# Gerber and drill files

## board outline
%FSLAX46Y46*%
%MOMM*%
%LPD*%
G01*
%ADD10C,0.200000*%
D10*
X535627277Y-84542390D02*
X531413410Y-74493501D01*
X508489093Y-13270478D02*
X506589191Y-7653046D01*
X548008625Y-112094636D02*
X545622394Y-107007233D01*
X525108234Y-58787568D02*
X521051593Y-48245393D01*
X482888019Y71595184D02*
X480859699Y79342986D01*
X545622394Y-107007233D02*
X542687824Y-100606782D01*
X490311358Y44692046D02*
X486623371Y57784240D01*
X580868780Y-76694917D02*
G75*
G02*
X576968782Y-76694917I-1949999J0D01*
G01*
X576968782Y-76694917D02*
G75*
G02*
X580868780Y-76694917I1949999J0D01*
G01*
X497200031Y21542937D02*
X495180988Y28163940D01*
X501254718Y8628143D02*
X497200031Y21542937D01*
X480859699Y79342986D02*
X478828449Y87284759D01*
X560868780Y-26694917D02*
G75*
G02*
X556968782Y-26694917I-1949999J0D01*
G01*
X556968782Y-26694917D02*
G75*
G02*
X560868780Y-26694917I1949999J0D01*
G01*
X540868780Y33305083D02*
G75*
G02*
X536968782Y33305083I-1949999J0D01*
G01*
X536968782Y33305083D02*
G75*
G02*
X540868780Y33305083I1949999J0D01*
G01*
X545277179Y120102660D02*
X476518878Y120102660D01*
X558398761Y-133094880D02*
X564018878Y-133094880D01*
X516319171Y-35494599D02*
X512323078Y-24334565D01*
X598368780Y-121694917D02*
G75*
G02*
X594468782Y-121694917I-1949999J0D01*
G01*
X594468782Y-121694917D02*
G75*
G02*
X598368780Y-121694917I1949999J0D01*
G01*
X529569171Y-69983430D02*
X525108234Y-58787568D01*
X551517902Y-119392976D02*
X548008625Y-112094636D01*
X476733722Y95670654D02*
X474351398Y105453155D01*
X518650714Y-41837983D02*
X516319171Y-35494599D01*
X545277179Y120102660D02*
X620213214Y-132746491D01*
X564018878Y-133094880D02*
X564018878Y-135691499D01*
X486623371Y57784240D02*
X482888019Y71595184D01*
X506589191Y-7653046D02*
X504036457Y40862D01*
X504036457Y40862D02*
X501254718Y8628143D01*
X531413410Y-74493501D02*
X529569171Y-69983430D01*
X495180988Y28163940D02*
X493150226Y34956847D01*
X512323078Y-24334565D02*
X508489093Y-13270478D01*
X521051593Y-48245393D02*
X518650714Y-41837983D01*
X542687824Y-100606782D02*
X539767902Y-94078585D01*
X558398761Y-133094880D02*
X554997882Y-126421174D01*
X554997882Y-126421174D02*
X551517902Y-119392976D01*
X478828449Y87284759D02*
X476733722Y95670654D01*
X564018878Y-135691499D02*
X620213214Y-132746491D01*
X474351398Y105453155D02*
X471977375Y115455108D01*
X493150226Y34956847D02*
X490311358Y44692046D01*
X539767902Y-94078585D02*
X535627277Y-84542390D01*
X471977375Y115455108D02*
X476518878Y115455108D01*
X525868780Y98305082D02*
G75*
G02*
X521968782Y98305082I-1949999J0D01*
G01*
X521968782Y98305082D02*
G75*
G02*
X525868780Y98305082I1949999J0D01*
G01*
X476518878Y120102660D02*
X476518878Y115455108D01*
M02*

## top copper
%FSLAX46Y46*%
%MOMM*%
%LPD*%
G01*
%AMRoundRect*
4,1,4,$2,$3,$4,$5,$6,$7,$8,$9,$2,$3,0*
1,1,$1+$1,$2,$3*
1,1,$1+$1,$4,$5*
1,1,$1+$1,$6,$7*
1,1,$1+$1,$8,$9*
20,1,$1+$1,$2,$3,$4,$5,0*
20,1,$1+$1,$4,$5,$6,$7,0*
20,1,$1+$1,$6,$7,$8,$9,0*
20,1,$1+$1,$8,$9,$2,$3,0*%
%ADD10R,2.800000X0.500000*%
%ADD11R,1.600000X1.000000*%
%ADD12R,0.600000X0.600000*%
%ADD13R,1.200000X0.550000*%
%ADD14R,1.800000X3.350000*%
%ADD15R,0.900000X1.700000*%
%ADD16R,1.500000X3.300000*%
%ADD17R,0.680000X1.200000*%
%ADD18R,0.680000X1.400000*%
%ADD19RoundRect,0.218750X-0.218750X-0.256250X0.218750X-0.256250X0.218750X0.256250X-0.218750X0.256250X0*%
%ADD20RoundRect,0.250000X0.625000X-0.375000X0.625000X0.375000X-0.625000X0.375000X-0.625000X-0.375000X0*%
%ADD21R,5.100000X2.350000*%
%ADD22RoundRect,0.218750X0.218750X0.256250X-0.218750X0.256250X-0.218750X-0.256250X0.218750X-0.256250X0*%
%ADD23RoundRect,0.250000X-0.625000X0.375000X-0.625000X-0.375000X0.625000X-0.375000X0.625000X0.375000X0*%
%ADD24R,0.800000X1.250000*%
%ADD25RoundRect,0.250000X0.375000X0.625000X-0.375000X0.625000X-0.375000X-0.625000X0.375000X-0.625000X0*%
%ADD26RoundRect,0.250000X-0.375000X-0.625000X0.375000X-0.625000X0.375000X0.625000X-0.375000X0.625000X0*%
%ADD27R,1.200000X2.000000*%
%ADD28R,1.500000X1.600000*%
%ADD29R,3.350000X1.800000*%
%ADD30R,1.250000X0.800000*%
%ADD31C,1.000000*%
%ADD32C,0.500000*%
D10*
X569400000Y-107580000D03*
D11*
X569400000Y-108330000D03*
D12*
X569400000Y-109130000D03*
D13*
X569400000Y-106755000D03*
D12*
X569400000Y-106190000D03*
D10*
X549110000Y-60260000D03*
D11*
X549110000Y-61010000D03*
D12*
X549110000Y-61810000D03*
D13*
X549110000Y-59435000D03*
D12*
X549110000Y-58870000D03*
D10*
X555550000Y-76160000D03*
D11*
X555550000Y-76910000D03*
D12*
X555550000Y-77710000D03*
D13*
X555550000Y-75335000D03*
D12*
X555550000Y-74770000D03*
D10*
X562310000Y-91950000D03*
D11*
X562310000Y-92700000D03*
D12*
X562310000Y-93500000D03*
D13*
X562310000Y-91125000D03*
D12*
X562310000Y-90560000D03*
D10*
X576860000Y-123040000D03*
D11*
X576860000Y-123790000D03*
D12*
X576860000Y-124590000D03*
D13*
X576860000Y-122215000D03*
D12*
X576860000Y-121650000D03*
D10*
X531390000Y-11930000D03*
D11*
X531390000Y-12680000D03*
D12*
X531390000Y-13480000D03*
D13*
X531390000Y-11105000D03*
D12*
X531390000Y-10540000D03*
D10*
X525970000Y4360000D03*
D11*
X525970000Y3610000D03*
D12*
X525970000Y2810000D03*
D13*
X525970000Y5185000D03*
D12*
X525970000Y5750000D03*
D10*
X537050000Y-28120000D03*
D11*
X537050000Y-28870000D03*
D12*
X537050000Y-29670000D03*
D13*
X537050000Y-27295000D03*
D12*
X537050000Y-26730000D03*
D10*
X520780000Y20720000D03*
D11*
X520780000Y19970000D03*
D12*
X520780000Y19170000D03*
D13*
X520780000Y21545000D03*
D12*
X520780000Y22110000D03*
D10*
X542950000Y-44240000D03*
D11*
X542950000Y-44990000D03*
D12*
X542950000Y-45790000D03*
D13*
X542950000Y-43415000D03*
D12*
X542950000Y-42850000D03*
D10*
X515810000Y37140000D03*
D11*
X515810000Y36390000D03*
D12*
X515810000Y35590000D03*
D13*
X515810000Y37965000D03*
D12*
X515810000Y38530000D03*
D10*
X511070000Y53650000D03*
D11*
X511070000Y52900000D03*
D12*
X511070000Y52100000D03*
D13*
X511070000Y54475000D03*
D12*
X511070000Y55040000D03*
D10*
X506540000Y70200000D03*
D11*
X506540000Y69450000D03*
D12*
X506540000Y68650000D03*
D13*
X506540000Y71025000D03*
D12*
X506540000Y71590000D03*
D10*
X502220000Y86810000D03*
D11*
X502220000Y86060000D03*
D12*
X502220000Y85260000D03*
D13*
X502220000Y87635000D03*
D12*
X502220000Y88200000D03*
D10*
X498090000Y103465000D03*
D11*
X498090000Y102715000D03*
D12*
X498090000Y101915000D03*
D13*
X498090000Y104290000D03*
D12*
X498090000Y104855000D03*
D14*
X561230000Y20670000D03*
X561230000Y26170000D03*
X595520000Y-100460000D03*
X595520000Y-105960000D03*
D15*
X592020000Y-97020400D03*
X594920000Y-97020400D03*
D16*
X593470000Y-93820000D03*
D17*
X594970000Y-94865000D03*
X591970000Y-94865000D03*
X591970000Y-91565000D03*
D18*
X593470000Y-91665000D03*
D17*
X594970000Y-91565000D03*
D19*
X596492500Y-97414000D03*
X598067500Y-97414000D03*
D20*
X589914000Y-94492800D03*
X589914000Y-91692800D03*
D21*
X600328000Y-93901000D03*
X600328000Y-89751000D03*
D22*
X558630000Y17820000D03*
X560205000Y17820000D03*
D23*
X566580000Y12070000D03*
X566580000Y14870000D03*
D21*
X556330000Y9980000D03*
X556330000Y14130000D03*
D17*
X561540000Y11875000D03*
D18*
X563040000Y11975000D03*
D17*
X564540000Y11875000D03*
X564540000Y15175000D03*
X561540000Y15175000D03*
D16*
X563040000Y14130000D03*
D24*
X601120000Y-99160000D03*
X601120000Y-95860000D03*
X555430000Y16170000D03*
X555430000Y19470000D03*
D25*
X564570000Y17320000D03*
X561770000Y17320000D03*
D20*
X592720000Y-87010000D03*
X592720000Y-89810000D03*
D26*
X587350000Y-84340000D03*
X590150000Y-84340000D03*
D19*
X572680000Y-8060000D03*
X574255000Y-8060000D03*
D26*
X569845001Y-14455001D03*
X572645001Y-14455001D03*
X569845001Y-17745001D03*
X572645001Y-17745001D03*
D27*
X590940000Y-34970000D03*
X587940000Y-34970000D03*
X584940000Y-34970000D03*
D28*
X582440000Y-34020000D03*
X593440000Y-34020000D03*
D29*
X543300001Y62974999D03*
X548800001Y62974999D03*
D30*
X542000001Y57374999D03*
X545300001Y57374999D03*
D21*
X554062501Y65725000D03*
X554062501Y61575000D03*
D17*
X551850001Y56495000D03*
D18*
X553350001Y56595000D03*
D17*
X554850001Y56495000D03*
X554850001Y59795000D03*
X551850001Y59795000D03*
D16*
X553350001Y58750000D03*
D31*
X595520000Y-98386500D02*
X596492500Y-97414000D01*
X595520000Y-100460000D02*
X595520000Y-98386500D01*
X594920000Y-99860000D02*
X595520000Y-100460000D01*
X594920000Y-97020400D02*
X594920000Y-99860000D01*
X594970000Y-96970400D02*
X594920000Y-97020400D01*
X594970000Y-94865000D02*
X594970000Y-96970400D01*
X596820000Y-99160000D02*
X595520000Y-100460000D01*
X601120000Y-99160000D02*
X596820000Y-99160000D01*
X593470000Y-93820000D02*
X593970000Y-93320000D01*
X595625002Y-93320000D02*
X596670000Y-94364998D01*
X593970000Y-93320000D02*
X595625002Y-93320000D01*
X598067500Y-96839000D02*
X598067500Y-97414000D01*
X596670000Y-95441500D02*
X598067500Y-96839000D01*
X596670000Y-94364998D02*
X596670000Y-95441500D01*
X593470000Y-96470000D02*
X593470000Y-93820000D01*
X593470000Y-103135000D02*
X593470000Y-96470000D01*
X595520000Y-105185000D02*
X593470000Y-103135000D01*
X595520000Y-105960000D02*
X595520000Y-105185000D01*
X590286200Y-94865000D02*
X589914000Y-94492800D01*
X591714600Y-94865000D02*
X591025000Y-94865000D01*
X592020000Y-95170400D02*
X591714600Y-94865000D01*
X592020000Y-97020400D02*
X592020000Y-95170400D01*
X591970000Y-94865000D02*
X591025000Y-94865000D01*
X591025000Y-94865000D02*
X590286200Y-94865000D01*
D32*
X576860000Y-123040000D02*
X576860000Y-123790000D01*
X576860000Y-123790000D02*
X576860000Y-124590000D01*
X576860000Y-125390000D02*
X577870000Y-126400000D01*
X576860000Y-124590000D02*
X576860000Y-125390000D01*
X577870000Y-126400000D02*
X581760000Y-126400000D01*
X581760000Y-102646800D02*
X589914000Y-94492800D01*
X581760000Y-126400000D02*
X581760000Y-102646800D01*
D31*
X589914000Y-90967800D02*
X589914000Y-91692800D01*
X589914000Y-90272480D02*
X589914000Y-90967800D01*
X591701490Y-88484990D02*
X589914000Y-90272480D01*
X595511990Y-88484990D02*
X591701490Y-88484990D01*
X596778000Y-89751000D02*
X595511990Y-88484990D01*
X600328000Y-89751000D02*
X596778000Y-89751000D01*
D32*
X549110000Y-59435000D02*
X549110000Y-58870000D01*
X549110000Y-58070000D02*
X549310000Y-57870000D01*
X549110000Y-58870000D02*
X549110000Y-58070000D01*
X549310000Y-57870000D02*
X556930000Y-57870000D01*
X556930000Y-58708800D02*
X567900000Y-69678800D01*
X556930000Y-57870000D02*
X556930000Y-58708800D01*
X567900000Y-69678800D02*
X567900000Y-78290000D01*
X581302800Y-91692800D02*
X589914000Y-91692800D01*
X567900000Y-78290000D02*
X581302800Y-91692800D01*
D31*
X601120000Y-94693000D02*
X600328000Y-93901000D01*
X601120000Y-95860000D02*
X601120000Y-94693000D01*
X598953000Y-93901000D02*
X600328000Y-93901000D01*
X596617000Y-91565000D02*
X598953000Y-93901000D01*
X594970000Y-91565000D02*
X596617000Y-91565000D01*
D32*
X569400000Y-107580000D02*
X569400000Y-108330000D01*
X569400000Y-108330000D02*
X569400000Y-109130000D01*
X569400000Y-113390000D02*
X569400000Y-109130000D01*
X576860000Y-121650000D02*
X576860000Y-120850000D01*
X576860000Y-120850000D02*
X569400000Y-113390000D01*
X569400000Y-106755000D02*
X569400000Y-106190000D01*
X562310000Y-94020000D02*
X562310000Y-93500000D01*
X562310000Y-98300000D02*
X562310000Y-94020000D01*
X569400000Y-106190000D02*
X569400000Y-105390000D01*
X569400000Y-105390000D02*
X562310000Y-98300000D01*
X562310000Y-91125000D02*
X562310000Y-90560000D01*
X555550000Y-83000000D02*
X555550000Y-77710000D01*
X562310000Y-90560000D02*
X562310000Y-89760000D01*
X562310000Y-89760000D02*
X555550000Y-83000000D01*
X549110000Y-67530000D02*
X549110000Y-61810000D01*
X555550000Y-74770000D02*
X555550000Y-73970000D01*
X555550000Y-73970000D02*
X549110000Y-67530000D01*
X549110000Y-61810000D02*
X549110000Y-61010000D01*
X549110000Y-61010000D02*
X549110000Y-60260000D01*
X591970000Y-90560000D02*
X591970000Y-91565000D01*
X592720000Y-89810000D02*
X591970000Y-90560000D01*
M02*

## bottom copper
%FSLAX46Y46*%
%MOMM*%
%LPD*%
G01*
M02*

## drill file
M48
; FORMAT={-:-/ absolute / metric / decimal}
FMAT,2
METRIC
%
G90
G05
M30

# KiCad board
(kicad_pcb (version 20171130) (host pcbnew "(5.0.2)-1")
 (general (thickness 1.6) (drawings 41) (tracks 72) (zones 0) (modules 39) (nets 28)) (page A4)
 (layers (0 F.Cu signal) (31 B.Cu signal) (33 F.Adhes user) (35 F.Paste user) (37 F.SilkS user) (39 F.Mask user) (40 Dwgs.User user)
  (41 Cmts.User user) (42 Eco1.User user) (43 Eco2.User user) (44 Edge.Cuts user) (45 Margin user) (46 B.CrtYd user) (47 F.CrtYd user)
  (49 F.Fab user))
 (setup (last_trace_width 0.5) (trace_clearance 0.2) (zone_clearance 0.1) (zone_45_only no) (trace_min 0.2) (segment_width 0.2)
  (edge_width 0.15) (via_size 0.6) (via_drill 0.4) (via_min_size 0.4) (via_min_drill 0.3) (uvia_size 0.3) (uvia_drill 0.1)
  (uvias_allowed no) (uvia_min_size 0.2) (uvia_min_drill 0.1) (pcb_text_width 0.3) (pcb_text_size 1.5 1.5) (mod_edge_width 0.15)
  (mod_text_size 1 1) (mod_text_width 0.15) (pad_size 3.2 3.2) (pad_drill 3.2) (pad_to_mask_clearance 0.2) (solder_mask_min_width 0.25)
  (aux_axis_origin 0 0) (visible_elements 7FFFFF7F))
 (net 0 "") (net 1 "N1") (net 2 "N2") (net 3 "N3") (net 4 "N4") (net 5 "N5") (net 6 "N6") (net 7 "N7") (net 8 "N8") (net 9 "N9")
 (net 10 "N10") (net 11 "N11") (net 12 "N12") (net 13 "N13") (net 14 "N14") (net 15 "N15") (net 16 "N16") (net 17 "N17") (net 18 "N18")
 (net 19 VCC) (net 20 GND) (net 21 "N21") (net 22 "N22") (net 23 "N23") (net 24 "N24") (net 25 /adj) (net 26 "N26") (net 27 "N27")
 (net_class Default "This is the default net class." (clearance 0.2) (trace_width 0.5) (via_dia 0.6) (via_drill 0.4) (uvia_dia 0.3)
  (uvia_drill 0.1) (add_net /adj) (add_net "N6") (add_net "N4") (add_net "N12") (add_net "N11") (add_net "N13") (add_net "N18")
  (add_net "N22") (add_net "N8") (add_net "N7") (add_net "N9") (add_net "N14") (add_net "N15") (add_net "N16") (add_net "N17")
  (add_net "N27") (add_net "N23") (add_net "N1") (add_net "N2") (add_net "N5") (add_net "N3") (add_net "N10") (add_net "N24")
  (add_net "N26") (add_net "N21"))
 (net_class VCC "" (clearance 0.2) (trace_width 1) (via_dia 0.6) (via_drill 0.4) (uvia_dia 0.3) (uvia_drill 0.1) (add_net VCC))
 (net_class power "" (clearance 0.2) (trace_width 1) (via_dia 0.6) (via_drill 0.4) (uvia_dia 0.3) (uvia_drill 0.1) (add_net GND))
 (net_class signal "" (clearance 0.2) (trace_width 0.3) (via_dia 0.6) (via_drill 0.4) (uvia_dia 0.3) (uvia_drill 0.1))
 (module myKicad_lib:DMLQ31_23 (layer F.Cu) (at 569.4 107.58 180)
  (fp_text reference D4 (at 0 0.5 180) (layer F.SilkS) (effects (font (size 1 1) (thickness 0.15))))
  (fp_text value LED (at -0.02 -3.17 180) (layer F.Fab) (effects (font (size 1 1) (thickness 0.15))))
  (pad 2 smd rect (at 0 0 180) (size 2.8 0.5) (layers F.Cu F.Paste F.Mask) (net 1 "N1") (zone_connect 2))
  (pad 2 smd rect (at 0 -0.75 180) (size 1.6 1) (layers F.Cu F.Paste F.Mask) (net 1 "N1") (zone_connect 2))
  (pad 2 smd rect (at 0 -1.55 180) (size 0.6 0.6) (layers F.Cu F.Paste F.Mask) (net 1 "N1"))
  (pad 1 smd rect (at 0 0.825 180) (size 1.2 0.55) (layers F.Cu F.Paste F.Mask) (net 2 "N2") (zone_connect 2))
  (pad 1 smd rect (at 0 1.39 180) (size 0.6 0.6) (layers F.Cu F.Paste F.Mask) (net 2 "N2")))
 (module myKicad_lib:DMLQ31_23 (layer F.Cu) (at 549.11 60.26 180)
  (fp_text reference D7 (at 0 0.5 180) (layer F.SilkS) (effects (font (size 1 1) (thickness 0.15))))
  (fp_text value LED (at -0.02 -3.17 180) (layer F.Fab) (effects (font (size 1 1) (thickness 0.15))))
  (pad 2 smd rect (at 0 0 180) (size 2.8 0.5) (layers F.Cu F.Paste F.Mask) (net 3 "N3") (zone_connect 2))
  (pad 2 smd rect (at 0 -0.75 180) (size 1.6 1) (layers F.Cu F.Paste F.Mask) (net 3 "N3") (zone_connect 2))
  (pad 2 smd rect (at 0 -1.55 180) (size 0.6 0.6) (layers F.Cu F.Paste F.Mask) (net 3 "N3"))
  (pad 1 smd rect (at 0 0.825 180) (size 1.2 0.55) (layers F.Cu F.Paste F.Mask) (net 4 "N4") (zone_connect 2))
  (pad 1 smd rect (at 0 1.39 180) (size 0.6 0.6) (layers F.Cu F.Paste F.Mask) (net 4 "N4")))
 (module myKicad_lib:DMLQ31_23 (layer F.Cu) (at 555.55 76.16 180)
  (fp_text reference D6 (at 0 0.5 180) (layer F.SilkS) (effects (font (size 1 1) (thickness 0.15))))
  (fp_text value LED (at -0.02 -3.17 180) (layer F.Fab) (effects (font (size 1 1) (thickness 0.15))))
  (pad 2 smd rect (at 0 0 180) (size 2.8 0.5) (layers F.Cu F.Paste F.Mask) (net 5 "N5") (zone_connect 2))
  (pad 2 smd rect (at 0 -0.75 180) (size 1.6 1) (layers F.Cu F.Paste F.Mask) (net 5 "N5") (zone_connect 2))
  (pad 2 smd rect (at 0 -1.55 180) (size 0.6 0.6) (layers F.Cu F.Paste F.Mask) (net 5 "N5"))
  (pad 1 smd rect (at 0 0.825 180) (size 1.2 0.55) (layers F.Cu F.Paste F.Mask) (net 3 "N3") (zone_connect 2))
  (pad 1 smd rect (at 0 1.39 180) (size 0.6 0.6) (layers F.Cu F.Paste F.Mask) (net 3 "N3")))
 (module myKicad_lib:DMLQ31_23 (layer F.Cu) (at 562.31 91.95 180)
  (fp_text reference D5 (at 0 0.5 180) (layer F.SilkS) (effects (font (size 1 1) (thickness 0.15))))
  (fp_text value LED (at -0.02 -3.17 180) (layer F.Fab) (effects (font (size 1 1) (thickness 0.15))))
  (pad 2 smd rect (at 0 0 180) (size 2.8 0.5) (layers F.Cu F.Paste F.Mask) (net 2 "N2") (zone_connect 2))
  (pad 2 smd rect (at 0 -0.75 180) (size 1.6 1) (layers F.Cu F.Paste F.Mask) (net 2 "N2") (zone_connect 2))
  (pad 2 smd rect (at 0 -1.55 180) (size 0.6 0.6) (layers F.Cu F.Paste F.Mask) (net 2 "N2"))
  (pad 1 smd rect (at 0 0.825 180) (size 1.2 0.55) (layers F.Cu F.Paste F.Mask) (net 5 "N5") (zone_connect 2))
  (pad 1 smd rect (at 0 1.39 180) (size 0.6 0.6) (layers F.Cu F.Paste F.Mask) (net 5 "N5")))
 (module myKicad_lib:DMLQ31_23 (layer F.Cu) (at 576.86 123.04 180)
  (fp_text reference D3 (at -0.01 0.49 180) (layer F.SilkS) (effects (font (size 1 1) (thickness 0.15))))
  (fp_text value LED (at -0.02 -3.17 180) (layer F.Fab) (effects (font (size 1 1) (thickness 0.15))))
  (pad 2 smd rect (at 0 0 180) (size 2.8 0.5) (layers F.Cu F.Paste F.Mask) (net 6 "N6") (zone_connect 2))
  (pad 2 smd rect (at 0 -0.75 180) (size 1.6 1) (layers F.Cu F.Paste F.Mask) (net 6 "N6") (zone_connect 2))
  (pad 2 smd rect (at 0 -1.55 180) (size 0.6 0.6) (layers F.Cu F.Paste F.Mask) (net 6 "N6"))
  (pad 1 smd rect (at 0 0.825 180) (size 1.2 0.55) (layers F.Cu F.Paste F.Mask) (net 1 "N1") (zone_connect 2))
  (pad 1 smd rect (at 0 1.39 180) (size 0.6 0.6) (layers F.Cu F.Paste F.Mask) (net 1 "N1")))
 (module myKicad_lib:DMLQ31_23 (layer F.Cu) (at 531.39 11.93 180)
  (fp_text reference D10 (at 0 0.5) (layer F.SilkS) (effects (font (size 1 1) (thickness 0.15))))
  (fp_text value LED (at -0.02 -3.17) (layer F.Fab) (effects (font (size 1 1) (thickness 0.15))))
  (pad 2 smd rect (at 0 0 180) (size 2.8 0.5) (layers F.Cu F.Paste F.Mask) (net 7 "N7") (zone_connect 2))
  (pad 2 smd rect (at 0 -0.75 180) (size 1.6 1) (layers F.Cu F.Paste F.Mask) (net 7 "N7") (zone_connect 2))
  (pad 2 smd rect (at 0 -1.55 180) (size 0.6 0.6) (layers F.Cu F.Paste F.Mask) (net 7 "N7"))
  (pad 1 smd rect (at 0 0.825 180) (size 1.2 0.55) (layers F.Cu F.Paste F.Mask) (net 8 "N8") (zone_connect 2))
  (pad 1 smd rect (at 0 1.39 180) (size 0.6 0.6) (layers F.Cu F.Paste F.Mask) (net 8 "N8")))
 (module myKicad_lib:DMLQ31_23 (layer F.Cu) (at 525.97 -4.36 180)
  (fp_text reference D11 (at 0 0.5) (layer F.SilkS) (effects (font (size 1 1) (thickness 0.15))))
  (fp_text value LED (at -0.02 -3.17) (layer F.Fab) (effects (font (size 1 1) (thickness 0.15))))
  (pad 2 smd rect (at 0 0 180) (size 2.8 0.5) (layers F.Cu F.Paste F.Mask) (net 8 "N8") (zone_connect 2))
  (pad 2 smd rect (at 0 -0.75 180) (size 1.6 1) (layers F.Cu F.Paste F.Mask) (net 8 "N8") (zone_connect 2))
  (pad 2 smd rect (at 0 -1.55 180) (size 0.6 0.6) (layers F.Cu F.Paste F.Mask) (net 8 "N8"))
  (pad 1 smd rect (at 0 0.825 180) (size 1.2 0.55) (layers F.Cu F.Paste F.Mask) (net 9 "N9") (zone_connect 2))
  (pad 1 smd rect (at 0 1.39 180) (size 0.6 0.6) (layers F.Cu F.Paste F.Mask) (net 9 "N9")))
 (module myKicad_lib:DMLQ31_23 (layer F.Cu) (at 537.05 28.12 180)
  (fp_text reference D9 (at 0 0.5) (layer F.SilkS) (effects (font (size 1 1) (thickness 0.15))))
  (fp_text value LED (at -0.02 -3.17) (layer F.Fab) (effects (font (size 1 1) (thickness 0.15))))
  (pad 2 smd rect (at 0 0 180) (size 2.8 0.5) (layers F.Cu F.Paste F.Mask) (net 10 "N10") (zone_connect 2))
  (pad 2 smd rect (at 0 -0.75 180) (size 1.6 1) (layers F.Cu F.Paste F.Mask) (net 10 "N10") (zone_connect 2))
  (pad 2 smd rect (at 0 -1.55 180) (size 0.6 0.6) (layers F.Cu F.Paste F.Mask) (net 10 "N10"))
  (pad 1 smd rect (at 0 0.825 180) (size 1.2 0.55) (layers F.Cu F.Paste F.Mask) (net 7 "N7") (zone_connect 2))
  (pad 1 smd rect (at 0 1.39 180) (size 0.6 0.6) (layers F.Cu F.Paste F.Mask) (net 7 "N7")))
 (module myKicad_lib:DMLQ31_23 (layer F.Cu) (at 520.78 -20.72 180)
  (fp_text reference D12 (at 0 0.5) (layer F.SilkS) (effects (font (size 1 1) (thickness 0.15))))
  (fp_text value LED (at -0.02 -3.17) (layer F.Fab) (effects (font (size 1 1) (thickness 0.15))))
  (pad 2 smd rect (at 0 0 180) (size 2.8 0.5) (layers F.Cu F.Paste F.Mask) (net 9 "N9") (zone_connect 2))
  (pad 2 smd rect (at 0 -0.75 180) (size 1.6 1) (layers F.Cu F.Paste F.Mask) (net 9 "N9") (zone_connect 2))
  (pad 2 smd rect (at 0 -1.55 180) (size 0.6 0.6) (layers F.Cu F.Paste F.Mask) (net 9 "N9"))
  (pad 1 smd rect (at 0 0.825 180) (size 1.2 0.55) (layers F.Cu F.Paste F.Mask) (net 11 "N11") (zone_connect 2))
  (pad 1 smd rect (at 0 1.39 180) (size 0.6 0.6) (layers F.Cu F.Paste F.Mask) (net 11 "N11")))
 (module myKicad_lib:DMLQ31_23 (layer F.Cu) (at 542.95 44.24 180)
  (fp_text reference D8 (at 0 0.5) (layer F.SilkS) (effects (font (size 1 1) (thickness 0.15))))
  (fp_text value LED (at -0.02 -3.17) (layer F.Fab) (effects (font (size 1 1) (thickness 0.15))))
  (pad 2 smd rect (at 0 0 180) (size 2.8 0.5) (layers F.Cu F.Paste F.Mask) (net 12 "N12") (zone_connect 2))
  (pad 2 smd rect (at 0 -0.75 180) (size 1.6 1) (layers F.Cu F.Paste F.Mask) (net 12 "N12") (zone_connect 2))
  (pad 2 smd rect (at 0 -1.55 180) (size 0.6 0.6) (layers F.Cu F.Paste F.Mask) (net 12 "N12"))
  (pad 1 smd rect (at 0 0.825 180) (size 1.2 0.55) (layers F.Cu F.Paste F.Mask) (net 10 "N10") (zone_connect 2))
  (pad 1 smd rect (at 0 1.39 180) (size 0.6 0.6) (layers F.Cu F.Paste F.Mask) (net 10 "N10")))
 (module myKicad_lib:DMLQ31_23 (layer F.Cu) (at 515.81 -37.14 180)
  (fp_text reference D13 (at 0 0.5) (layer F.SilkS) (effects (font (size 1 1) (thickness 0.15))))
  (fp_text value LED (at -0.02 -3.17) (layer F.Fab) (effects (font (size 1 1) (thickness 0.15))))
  (pad 2 smd rect (at 0 0 180) (size 2.8 0.5) (layers F.Cu F.Paste F.Mask) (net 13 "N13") (zone_connect 2))
  (pad 2 smd rect (at 0 -0.75 180) (size 1.6 1) (layers F.Cu F.Paste F.Mask) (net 13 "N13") (zone_connect 2))
  (pad 2 smd rect (at 0 -1.55 180) (size 0.6 0.6) (layers F.Cu F.Paste F.Mask) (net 13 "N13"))
  (pad 1 smd rect (at 0 0.825 180) (size 1.2 0.55) (layers F.Cu F.Paste F.Mask) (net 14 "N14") (zone_connect 2))
  (pad 1 smd rect (at 0 1.39 180) (size 0.6 0.6) (layers F.Cu F.Paste F.Mask) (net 14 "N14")))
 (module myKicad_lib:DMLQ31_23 (layer F.Cu) (at 511.07 -53.65 180)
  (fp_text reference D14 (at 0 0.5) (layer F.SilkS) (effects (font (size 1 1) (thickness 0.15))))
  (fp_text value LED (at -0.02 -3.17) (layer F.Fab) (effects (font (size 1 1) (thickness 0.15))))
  (pad 2 smd rect (at 0 0 180) (size 2.8 0.5) (layers F.Cu F.Paste F.Mask) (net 14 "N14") (zone_connect 2))
  (pad 2 smd rect (at 0 -0.75 180) (size 1.6 1) (layers F.Cu F.Paste F.Mask) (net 14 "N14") (zone_connect 2))
  (pad 2 smd rect (at 0 -1.55 180) (size 0.6 0.6) (layers F.Cu F.Paste F.Mask) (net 14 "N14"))
  (pad 1 smd rect (at 0 0.825 180) (size 1.2 0.55) (layers F.Cu F.Paste F.Mask) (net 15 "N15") (zone_connect 2))
  (pad 1 smd rect (at 0 1.39 180) (size 0.6 0.6) (layers F.Cu F.Paste F.Mask) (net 15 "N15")))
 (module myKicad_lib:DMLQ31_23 (layer F.Cu) (at 506.54 -70.2 180)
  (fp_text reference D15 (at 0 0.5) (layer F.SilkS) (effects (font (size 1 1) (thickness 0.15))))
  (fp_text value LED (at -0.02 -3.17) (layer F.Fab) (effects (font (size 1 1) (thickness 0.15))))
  (pad 2 smd rect (at 0 0 180) (size 2.8 0.5) (layers F.Cu F.Paste F.Mask) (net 15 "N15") (zone_connect 2))
  (pad 2 smd rect (at 0 -0.75 180) (size 1.6 1) (layers F.Cu F.Paste F.Mask) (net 15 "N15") (zone_connect 2))
  (pad 2 smd rect (at 0 -1.55 180) (size 0.6 0.6) (layers F.Cu F.Paste F.Mask) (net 15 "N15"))
  (pad 1 smd rect (at 0 0.825 180) (size 1.2 0.55) (layers F.Cu F.Paste F.Mask) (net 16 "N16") (zone_connect 2))
  (pad 1 smd rect (at 0 1.39 180) (size 0.6 0.6) (layers F.Cu F.Paste F.Mask) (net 16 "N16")))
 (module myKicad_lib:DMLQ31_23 (layer F.Cu) (at 502.22 -86.81 180)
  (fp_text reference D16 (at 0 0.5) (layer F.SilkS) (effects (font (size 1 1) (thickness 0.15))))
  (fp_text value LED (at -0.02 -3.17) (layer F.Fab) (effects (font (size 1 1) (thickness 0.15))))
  (pad 2 smd rect (at 0 0 180) (size 2.8 0.5) (layers F.Cu F.Paste F.Mask) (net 16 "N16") (zone_connect 2))
  (pad 2 smd rect (at 0 -0.75 180) (size 1.6 1) (layers F.Cu F.Paste F.Mask) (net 16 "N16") (zone_connect 2))
  (pad 2 smd rect (at 0 -1.55 180) (size 0.6 0.6) (layers F.Cu F.Paste F.Mask) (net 16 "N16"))
  (pad 1 smd rect (at 0 0.825 180) (size 1.2 0.55) (layers F.Cu F.Paste F.Mask) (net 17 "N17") (zone_connect 2))
  (pad 1 smd rect (at 0 1.39 180) (size 0.6 0.6) (layers F.Cu F.Paste F.Mask) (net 17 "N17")))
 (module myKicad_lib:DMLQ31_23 (layer F.Cu) (at 498.09 -103.465 180)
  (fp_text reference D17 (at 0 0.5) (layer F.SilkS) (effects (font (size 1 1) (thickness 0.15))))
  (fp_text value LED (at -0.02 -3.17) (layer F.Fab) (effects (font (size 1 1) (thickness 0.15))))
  (pad 2 smd rect (at 0 0 180) (size 2.8 0.5) (layers F.Cu F.Paste F.Mask) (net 17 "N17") (zone_connect 2))
  (pad 2 smd rect (at 0 -0.75 180) (size 1.6 1) (layers F.Cu F.Paste F.Mask) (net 17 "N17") (zone_connect 2))
  (pad 2 smd rect (at 0 -1.55 180) (size 0.6 0.6) (layers F.Cu F.Paste F.Mask) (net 17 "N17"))
  (pad 1 smd rect (at 0 0.825 180) (size 1.2 0.55) (layers F.Cu F.Paste F.Mask) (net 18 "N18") (zone_connect 2))
  (pad 1 smd rect (at 0 1.39 180) (size 0.6 0.6) (layers F.Cu F.Paste F.Mask) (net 18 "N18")))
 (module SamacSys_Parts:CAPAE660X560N (layer F.Cu) (at 561.23 -23.42 90)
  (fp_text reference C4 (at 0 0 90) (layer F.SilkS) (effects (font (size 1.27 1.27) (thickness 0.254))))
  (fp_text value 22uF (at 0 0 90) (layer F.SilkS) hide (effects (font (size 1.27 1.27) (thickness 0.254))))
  (pad 1 smd rect (at -2.75 0 180) (size 1.8 3.35) (layers F.Cu F.Paste F.Mask) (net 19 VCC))
  (pad 2 smd rect (at 2.75 0 180) (size 1.8 3.35) (layers F.Cu F.Paste F.Mask) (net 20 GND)))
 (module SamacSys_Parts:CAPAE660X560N (layer F.Cu) (at 595.52 103.21 270)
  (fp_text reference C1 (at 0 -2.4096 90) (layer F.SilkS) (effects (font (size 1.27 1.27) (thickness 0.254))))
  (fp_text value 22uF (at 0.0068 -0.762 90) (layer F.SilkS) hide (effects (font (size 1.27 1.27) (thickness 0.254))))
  (pad 1 smd rect (at -2.75 0) (size 1.8 3.35) (layers F.Cu F.Paste F.Mask) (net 19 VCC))
  (pad 2 smd rect (at 2.75 0) (size 1.8 3.35) (layers F.Cu F.Paste F.Mask) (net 20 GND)))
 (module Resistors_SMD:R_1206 (layer F.Cu) (at 593.47 97.0204)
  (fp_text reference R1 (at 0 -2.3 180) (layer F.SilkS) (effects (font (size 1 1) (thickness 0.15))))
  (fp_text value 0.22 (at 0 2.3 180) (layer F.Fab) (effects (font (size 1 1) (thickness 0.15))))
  (pad 1 smd rect (at -1.45 0) (size 0.9 1.7) (layers F.Cu F.Paste F.Mask) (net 6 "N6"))
  (pad 2 smd rect (at 1.45 0) (size 0.9 1.7) (layers F.Cu F.Paste F.Mask) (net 19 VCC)))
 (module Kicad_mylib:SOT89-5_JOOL (layer F.Cu) (at 593.47 93.215 180)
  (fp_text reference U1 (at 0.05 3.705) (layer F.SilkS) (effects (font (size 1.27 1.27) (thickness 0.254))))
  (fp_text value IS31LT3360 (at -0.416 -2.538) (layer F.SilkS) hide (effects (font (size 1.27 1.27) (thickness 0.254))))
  (pad 2 smd rect (at 0 -0.605 180) (size 1.5 3.3) (layers F.Cu F.Paste F.Mask) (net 20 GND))
  (pad 5 smd rect (at -1.5 -1.65 180) (size 0.68 1.2) (layers F.Cu F.Paste F.Mask) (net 19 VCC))
  (pad 4 smd rect (at 1.5 -1.65 180) (size 0.68 1.2) (layers F.Cu F.Paste F.Mask) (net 6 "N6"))
  (pad 3 smd rect (at 1.5 1.65 180) (size 0.68 1.2) (layers F.Cu F.Paste F.Mask) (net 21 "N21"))
  (pad 2 smd rect (at 0 1.55 180) (size 0.68 1.4) (layers F.Cu F.Paste F.Mask) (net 20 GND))
  (pad 1 smd rect (at -1.5 1.65 180) (size 0.68 1.2) (layers F.Cu F.Paste F.Mask) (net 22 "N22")))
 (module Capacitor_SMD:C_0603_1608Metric (layer F.Cu) (at 597.28 97.414)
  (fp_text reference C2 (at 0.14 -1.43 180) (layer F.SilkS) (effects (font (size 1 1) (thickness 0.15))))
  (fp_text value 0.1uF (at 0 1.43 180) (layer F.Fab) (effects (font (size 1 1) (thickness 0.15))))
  (pad 1 smd roundrect (at -0.7875 0) (size 0.875 0.95) (layers F.Cu F.Paste F.Mask) (roundrect_rratio 0.25) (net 19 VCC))
  (pad 2 smd roundrect (at 0.7875 0) (size 0.875 0.95) (layers F.Cu F.Paste F.Mask) (roundrect_rratio 0.25) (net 20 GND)))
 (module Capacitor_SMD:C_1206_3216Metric (layer F.Cu) (at 589.914 93.0928 90)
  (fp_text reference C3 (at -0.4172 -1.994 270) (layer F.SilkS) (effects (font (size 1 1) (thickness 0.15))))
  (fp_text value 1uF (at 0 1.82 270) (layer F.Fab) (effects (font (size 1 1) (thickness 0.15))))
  (pad 1 smd roundrect (at -1.4 0 90) (size 1.25 1.75) (layers F.Cu F.Paste F.Mask) (roundrect_rratio 0.2) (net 6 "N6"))
  (pad 2 smd roundrect (at 1.4 0 90) (size 1.25 1.75) (layers F.Cu F.Paste F.Mask) (roundrect_rratio 0.2) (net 4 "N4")))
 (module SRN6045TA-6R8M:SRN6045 (layer F.Cu) (at 600.328 91.826 180)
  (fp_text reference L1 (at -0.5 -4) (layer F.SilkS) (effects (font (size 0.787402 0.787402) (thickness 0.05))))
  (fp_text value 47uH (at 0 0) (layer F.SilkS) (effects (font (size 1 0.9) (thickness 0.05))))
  (pad 1 smd rect (at 0 -2.075 180) (size 5.1 2.35) (layers F.Cu F.Paste F.Mask) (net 22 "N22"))
  (pad 2 smd rect (at 0 2.075 180) (size 5.1 2.35) (layers F.Cu F.Paste F.Mask) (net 4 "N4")))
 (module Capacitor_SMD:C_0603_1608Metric (layer F.Cu) (at 559.4175 -17.82 180)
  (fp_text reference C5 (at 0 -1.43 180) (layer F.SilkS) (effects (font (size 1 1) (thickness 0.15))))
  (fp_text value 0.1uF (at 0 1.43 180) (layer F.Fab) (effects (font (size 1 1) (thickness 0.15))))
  (pad 2 smd roundrect (at 0.7875 0 180) (size 0.875 0.95) (layers F.Cu F.Paste F.Mask) (roundrect_rratio 0.25) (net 20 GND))
  (pad 1 smd roundrect (at -0.7875 0 180) (size 0.875 0.95) (layers F.Cu F.Paste F.Mask) (roundrect_rratio 0.25) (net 19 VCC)))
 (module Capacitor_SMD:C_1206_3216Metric (layer F.Cu) (at 566.58 -13.47 270)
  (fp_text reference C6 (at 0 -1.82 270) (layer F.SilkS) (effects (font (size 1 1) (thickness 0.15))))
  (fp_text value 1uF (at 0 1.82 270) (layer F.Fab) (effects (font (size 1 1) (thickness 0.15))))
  (pad 2 smd roundrect (at 1.4 0 270) (size 1.25 1.75) (layers F.Cu F.Paste F.Mask) (roundrect_rratio 0.2) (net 11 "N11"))
  (pad 1 smd roundrect (at -1.4 0 270) (size 1.25 1.75) (layers F.Cu F.Paste F.Mask) (roundrect_rratio 0.2) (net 12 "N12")))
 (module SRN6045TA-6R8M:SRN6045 (layer F.Cu) (at 556.33 -12.055)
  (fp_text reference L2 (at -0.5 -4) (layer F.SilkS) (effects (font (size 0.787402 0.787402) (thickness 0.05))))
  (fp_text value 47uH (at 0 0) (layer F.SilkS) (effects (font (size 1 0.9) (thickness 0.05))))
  (pad 2 smd rect (at 0 2.075) (size 5.1 2.35) (layers F.Cu F.Paste F.Mask) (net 11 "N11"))
  (pad 1 smd rect (at 0 -2.075) (size 5.1 2.35) (layers F.Cu F.Paste F.Mask) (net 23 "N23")))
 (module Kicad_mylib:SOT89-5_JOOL (layer F.Cu) (at 563.04 -13.525)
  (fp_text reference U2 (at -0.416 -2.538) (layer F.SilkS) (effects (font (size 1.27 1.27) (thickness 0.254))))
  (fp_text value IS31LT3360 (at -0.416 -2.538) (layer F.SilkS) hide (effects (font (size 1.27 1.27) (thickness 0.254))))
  (pad 1 smd rect (at -1.5 1.65) (size 0.68 1.2) (layers F.Cu F.Paste F.Mask) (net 23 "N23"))
  (pad 2 smd rect (at 0 1.55) (size 0.68 1.4) (layers F.Cu F.Paste F.Mask) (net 20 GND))
  (pad 3 smd rect (at 1.5 1.65) (size 0.68 1.2) (layers F.Cu F.Paste F.Mask) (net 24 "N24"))
  (pad 4 smd rect (at 1.5 -1.65) (size 0.68 1.2) (layers F.Cu F.Paste F.Mask) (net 12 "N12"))
  (pad 5 smd rect (at -1.5 -1.65) (size 0.68 1.2) (layers F.Cu F.Paste F.Mask) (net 19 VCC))
  (pad 2 smd rect (at 0 -0.605) (size 1.5 3.3) (layers F.Cu F.Paste F.Mask) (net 20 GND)))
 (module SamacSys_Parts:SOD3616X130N (layer F.Cu) (at 601.12 97.51 90)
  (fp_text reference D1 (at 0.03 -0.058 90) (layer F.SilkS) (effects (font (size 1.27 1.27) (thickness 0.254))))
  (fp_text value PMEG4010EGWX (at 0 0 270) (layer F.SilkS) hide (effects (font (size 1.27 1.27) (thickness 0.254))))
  (pad 1 smd rect (at -1.65 0 180) (size 0.8 1.25) (layers F.Cu F.Paste F.Mask) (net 19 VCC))
  (pad 2 smd rect (at 1.65 0 180) (size 0.8 1.25) (layers F.Cu F.Paste F.Mask) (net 22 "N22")))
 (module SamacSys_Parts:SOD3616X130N (layer F.Cu) (at 555.43 -17.82 270)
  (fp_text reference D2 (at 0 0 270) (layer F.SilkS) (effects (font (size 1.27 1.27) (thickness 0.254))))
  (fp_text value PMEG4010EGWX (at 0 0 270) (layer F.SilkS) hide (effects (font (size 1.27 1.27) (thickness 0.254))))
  (pad 2 smd rect (at 1.65 0) (size 0.8 1.25) (layers F.Cu F.Paste F.Mask) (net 23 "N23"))
  (pad 1 smd rect (at -1.65 0) (size 0.8 1.25) (layers F.Cu F.Paste F.Mask) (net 19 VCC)))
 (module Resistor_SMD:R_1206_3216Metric (layer F.Cu) (at 563.17 -17.32 180)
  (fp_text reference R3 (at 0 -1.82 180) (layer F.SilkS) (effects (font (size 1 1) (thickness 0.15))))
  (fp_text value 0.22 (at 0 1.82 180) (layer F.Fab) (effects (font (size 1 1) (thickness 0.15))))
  (pad 1 smd roundrect (at -1.4 0 180) (size 1.25 1.75) (layers F.Cu F.Paste F.Mask) (roundrect_rratio 0.2) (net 12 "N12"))
  (pad 2 smd roundrect (at 1.4 0 180) (size 1.25 1.75) (layers F.Cu F.Paste F.Mask) (roundrect_rratio 0.2) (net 19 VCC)))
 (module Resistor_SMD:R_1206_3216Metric (layer F.Cu) (at 592.72 88.41 90)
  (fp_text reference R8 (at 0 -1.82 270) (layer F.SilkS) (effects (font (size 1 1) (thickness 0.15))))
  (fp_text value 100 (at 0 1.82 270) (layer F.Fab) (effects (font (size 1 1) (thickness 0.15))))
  (pad 2 smd roundrect (at 1.4 0 90) (size 1.25 1.75) (layers F.Cu F.Paste F.Mask) (roundrect_rratio 0.2) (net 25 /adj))
  (pad 1 smd roundrect (at -1.4 0 90) (size 1.25 1.75) (layers F.Cu F.Paste F.Mask) (roundrect_rratio 0.2) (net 21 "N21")))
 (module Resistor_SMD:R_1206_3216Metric (layer F.Cu) (at 588.75 84.34)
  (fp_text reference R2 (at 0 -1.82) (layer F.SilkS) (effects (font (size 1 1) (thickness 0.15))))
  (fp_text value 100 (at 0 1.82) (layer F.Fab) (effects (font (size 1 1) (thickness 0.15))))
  (pad 1 smd roundrect (at -1.4 0) (size 1.25 1.75) (layers F.Cu F.Paste F.Mask) (roundrect_rratio 0.2) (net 24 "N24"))
  (pad 2 smd roundrect (at 1.4 0) (size 1.25 1.75) (layers F.Cu F.Paste F.Mask) (roundrect_rratio 0.2) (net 25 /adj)))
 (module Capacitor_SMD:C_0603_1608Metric (layer F.Cu) (at 573.4675 8.06)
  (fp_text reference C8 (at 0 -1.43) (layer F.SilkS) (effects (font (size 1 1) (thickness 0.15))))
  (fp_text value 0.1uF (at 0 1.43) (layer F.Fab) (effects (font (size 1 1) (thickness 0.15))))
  (pad 1 smd roundrect (at -0.7875 0) (size 0.875 0.95) (layers F.Cu F.Paste F.Mask) (roundrect_rratio 0.25) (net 19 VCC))
  (pad 2 smd roundrect (at 0.7875 0) (size 0.875 0.95) (layers F.Cu F.Paste F.Mask) (roundrect_rratio 0.25) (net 20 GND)))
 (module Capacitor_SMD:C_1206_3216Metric (layer F.Cu) (at 571.245001 14.455001)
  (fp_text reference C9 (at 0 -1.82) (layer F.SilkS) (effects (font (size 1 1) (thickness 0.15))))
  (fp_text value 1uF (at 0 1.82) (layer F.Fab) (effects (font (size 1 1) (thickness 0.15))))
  (pad 1 smd roundrect (at -1.4 0) (size 1.25 1.75) (layers F.Cu F.Paste F.Mask) (roundrect_rratio 0.2) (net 13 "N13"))
  (pad 2 smd roundrect (at 1.4 0) (size 1.25 1.75) (layers F.Cu F.Paste F.Mask) (roundrect_rratio 0.2) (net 18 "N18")))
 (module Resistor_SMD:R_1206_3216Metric (layer F.Cu) (at 571.245001 17.745001)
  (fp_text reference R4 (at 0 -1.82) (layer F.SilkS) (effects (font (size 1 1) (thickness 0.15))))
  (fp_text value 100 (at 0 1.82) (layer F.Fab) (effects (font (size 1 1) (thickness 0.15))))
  (pad 1 smd roundrect (at -1.4 0) (size 1.25 1.75) (layers F.Cu F.Paste F.Mask) (roundrect_rratio 0.2) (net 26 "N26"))
  (pad 2 smd roundrect (at 1.4 0) (size 1.25 1.75) (layers F.Cu F.Paste F.Mask) (roundrect_rratio 0.2) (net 25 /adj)))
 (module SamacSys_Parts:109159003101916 (layer F.Cu) (at 587.94 34.97)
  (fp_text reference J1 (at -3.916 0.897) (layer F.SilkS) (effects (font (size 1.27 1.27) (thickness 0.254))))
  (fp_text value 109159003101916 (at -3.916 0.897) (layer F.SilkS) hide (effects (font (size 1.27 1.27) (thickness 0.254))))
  (pad 1 smd rect (at 3 0) (size 1.2 2) (layers F.Cu F.Paste)) (pad 2 smd rect (at 0 0) (size 1.2 2) (layers F.Cu F.Paste))
  (pad 3 smd rect (at -3 0) (size 1.2 2) (layers F.Cu F.Paste))
  (pad 4 smd rect (at -5.5 -0.95) (size 1.5 1.6) (layers F.Cu F.Paste))
  (pad 5 smd rect (at 5.5 -0.95) (size 1.5 1.6) (layers F.Cu F.Paste)))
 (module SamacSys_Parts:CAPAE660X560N (layer F.Cu) (at 546.050001 -62.974999)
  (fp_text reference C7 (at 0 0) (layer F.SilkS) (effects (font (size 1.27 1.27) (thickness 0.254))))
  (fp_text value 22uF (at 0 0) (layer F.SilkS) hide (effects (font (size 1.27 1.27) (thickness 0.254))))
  (pad 1 smd rect (at -2.75 0 90) (size 1.8 3.35) (layers F.Cu F.Paste F.Mask) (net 19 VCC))
  (pad 2 smd rect (at 2.75 0 90) (size 1.8 3.35) (layers F.Cu F.Paste F.Mask) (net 20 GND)))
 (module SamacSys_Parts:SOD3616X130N (layer F.Cu) (at 543.650001 -57.374999)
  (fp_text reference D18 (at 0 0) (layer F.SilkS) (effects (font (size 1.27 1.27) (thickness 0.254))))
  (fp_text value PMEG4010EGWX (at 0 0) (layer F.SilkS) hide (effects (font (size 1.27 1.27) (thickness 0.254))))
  (pad 1 smd rect (at -1.65 0 90) (size 0.8 1.25) (layers F.Cu F.Paste F.Mask) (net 19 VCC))
  (pad 2 smd rect (at 1.65 0 90) (size 0.8 1.25) (layers F.Cu F.Paste F.Mask) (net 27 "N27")))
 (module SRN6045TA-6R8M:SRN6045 (layer F.Cu) (at 554.062501 -63.65)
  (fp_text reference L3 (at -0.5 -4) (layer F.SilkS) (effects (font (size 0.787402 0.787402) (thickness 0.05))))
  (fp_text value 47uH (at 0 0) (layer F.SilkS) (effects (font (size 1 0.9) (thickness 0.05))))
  (pad 1 smd rect (at 0 -2.075) (size 5.1 2.35) (layers F.Cu F.Paste F.Mask) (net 27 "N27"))
  (pad 2 smd rect (at 0 2.075) (size 5.1 2.35) (layers F.Cu F.Paste F.Mask) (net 18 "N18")))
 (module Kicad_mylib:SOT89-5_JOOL (layer F.Cu) (at 553.350001 -58.145)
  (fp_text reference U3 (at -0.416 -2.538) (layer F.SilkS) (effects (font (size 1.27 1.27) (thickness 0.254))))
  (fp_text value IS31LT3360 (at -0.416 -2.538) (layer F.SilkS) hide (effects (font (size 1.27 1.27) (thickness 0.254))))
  (pad 1 smd rect (at -1.5 1.65) (size 0.68 1.2) (layers F.Cu F.Paste F.Mask) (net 27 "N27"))
  (pad 2 smd rect (at 0 1.55) (size 0.68 1.4) (layers F.Cu F.Paste F.Mask) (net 20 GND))
  (pad 3 smd rect (at 1.5 1.65) (size 0.68 1.2) (layers F.Cu F.Paste F.Mask) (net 26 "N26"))
  (pad 4 smd rect (at 1.5 -1.65) (size 0.68 1.2) (layers F.Cu F.Paste F.Mask) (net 13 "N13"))
  (pad 5 smd rect (at -1.5 -1.65) (size 0.68 1.2) (layers F.Cu F.Paste F.Mask) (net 19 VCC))
  (pad 2 smd rect (at 0 -0.605) (size 1.5 3.3) (layers F.Cu F.Paste F.Mask) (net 20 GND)))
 (gr_line (start 535.627277 84.54239) (end 531.41341 74.493501) (layer Edge.Cuts) (width 0.2))
 (gr_line (start 508.489093 13.270478) (end 506.589191 7.653046) (layer Edge.Cuts) (width 0.2))
 (gr_line (start 548.008625 112.094636) (end 545.622394 107.007233) (layer Edge.Cuts) (width 0.2))
 (gr_line (start 525.108234 58.787568) (end 521.051593 48.245393) (layer Edge.Cuts) (width 0.2))
 (gr_line (start 482.888019 -71.595184) (end 480.859699 -79.342986) (layer Edge.Cuts) (width 0.2))
 (gr_line (start 545.622394 107.007233) (end 542.687824 100.606782) (layer Edge.Cuts) (width 0.2))
 (gr_line (start 490.311358 -44.692046) (end 486.623371 -57.78424) (layer Edge.Cuts) (width 0.2))
 (gr_circle (center 578.918781 76.694917) (end 580.86878 76.694917) (layer Edge.Cuts) (width 0.2))
 (gr_line (start 497.200031 -21.542937) (end 495.180988 -28.16394) (layer Edge.Cuts) (width 0.2))
 (gr_line (start 501.254718 -8.628143) (end 497.200031 -21.542937) (layer Edge.Cuts) (width 0.2))
 (gr_line (start 480.859699 -79.342986) (end 478.828449 -87.284759) (layer Edge.Cuts) (width 0.2))
 (gr_circle (center 558.918781 26.694917) (end 560.86878 26.694917) (layer Edge.Cuts) (width 0.2))
 (gr_circle (center 538.918781 -33.305083) (end 540.86878 -33.305083) (layer Edge.Cuts) (width 0.2))
 (gr_line (start 545.277179 -120.10266) (end 476.518878 -120.10266) (layer Edge.Cuts) (width 0.2))
 (gr_line (start 558.398761 133.09488) (end 564.018878 133.09488) (layer Edge.Cuts) (width 0.2))
 (gr_line (start 516.319171 35.494599) (end 512.323078 24.334565) (layer Edge.Cuts) (width 0.2))
 (gr_circle (center 596.418781 121.694917) (end 598.36878 121.694917) (layer Edge.Cuts) (width 0.2))
 (gr_line (start 529.569171 69.98343) (end 525.108234 58.787568) (layer Edge.Cuts) (width 0.2))
 (gr_line (start 551.517902 119.392976) (end 548.008625 112.094636) (layer Edge.Cuts) (width 0.2))
 (gr_line (start 476.733722 -95.670654) (end 474.351398 -105.453155) (layer Edge.Cuts) (width 0.2))
 (gr_line (start 518.650714 41.837983) (end 516.319171 35.494599) (layer Edge.Cuts) (width 0.2))
 (gr_line (start 545.277179 -120.10266) (end 620.213214 132.746491) (layer Edge.Cuts) (width 0.2))
 (gr_line (start 564.018878 133.09488) (end 564.018878 135.691499) (layer Edge.Cuts) (width 0.2))
 (gr_line (start 486.623371 -57.78424) (end 482.888019 -71.595184) (layer Edge.Cuts) (width 0.2))
 (gr_line (start 506.589191 7.653046) (end 504.036457 -0.040862) (layer Edge.Cuts) (width 0.2))
 (gr_line (start 504.036457 -0.040862) (end 501.254718 -8.628143) (layer Edge.Cuts) (width 0.2))
 (gr_line (start 531.41341 74.493501) (end 529.569171 69.98343) (layer Edge.Cuts) (width 0.2))
 (gr_line (start 495.180988 -28.16394) (end 493.150226 -34.956847) (layer Edge.Cuts) (width 0.2))
 (gr_line (start 512.323078 24.334565) (end 508.489093 13.270478) (layer Edge.Cuts) (width 0.2))
 (gr_line (start 521.051593 48.245393) (end 518.650714 41.837983) (layer Edge.Cuts) (width 0.2))
 (gr_line (start 542.687824 100.606782) (end 539.767902 94.078585) (layer Edge.Cuts) (width 0.2))
 (gr_line (start 558.398761 133.09488) (end 554.997882 126.421174) (layer Edge.Cuts) (width 0.2))
 (gr_line (start 554.997882 126.421174) (end 551.517902 119.392976) (layer Edge.Cuts) (width 0.2))
 (gr_line (start 478.828449 -87.284759) (end 476.733722 -95.670654) (layer Edge.Cuts) (width 0.2))
 (gr_line (start 564.018878 135.691499) (end 620.213214 132.746491) (layer Edge.Cuts) (width 0.2))
 (gr_line (start 474.351398 -105.453155) (end 471.977375 -115.455108) (layer Edge.Cuts) (width 0.2))
 (gr_line (start 493.150226 -34.956847) (end 490.311358 -44.692046) (layer Edge.Cuts) (width 0.2))
 (gr_line (start 539.767902 94.078585) (end 535.627277 84.54239) (layer Edge.Cuts) (width 0.2))
 (gr_line (start 471.977375 -115.455108) (end 476.518878 -115.455108) (layer Edge.Cuts) (width 0.2))
 (gr_circle (center 523.918781 -98.305082) (end 525.86878 -98.305082) (layer Edge.Cuts) (width 0.2))
 (gr_line (start 476.518878 -120.10266) (end 476.518878 -115.455108) (layer Edge.Cuts) (width 0.2))
 (segment (start 595.52 98.3865) (end 596.4925 97.414) (width 1) (layer F.Cu) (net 19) (status 20))
 (segment (start 595.52 100.46) (end 595.52 98.3865) (width 1) (layer F.Cu) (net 19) (status 10))
 (segment (start 594.92 99.86) (end 595.52 100.46) (width 1) (layer F.Cu) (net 19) (status 30))
 (segment (start 594.92 97.0204) (end 594.92 99.86) (width 1) (layer F.Cu) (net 19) (status 30))
 (segment (start 594.97 96.9704) (end 594.92 97.0204) (width 1) (layer F.Cu) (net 19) (status 30))
 (segment (start 594.97 94.865) (end 594.97 96.9704) (width 1) (layer F.Cu) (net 19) (status 30))
 (segment (start 596.82 99.16) (end 595.52 100.46) (width 1) (layer F.Cu) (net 19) (status 20))
 (segment (start 601.12 99.16) (end 596.82 99.16) (width 1) (layer F.Cu) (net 19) (status 10))
 (segment (start 593.47 93.82) (end 593.97 93.32) (width 1) (layer F.Cu) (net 20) (status 30))
 (segment (start 595.625002 93.32) (end 596.67 94.364998) (width 1) (layer F.Cu) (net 20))
 (segment (start 593.97 93.32) (end 595.625002 93.32) (width 1) (layer F.Cu) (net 20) (status 10))
 (segment (start 598.0675 96.839) (end 598.0675 97.414) (width 1) (layer F.Cu) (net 20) (status 20))
 (segment (start 596.67 95.4415) (end 598.0675 96.839) (width 1) (layer F.Cu) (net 20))
 (segment (start 596.67 94.364998) (end 596.67 95.4415) (width 1) (layer F.Cu) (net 20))
 (segment (start 593.47 96.47) (end 593.47 93.82) (width 1) (layer F.Cu) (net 20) (status 20))
 (segment (start 593.47 103.135) (end 593.47 96.47) (width 1) (layer F.Cu) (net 20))
 (segment (start 595.52 105.185) (end 593.47 103.135) (width 1) (layer F.Cu) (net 20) (status 10))
 (segment (start 595.52 105.96) (end 595.52 105.185) (width 1) (layer F.Cu) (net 20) (status 30))
 (segment (start 590.2862 94.865) (end 589.914 94.4928) (width 1) (layer F.Cu) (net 6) (status 30))
 (segment (start 591.7146 94.865) (end 591.025 94.865) (width 1) (layer F.Cu) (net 6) (status 10))
 (segment (start 592.02 95.1704) (end 591.7146 94.865) (width 1) (layer F.Cu) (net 6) (status 30))
 (segment (start 592.02 97.0204) (end 592.02 95.1704) (width 1) (layer F.Cu) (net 6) (status 30))
 (segment (start 591.97 94.865) (end 591.025 94.865) (width 1) (layer F.Cu) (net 6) (status 10))
 (segment (start 591.025 94.865) (end 590.2862 94.865) (width 1) (layer F.Cu) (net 6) (status 20))
 (segment (start 576.86 123.04) (end 576.86 123.79) (width 0.5) (layer F.Cu) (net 6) (status 30))
 (segment (start 576.86 123.79) (end 576.86 124.59) (width 0.5) (layer F.Cu) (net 6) (status 30))
 (segment (start 576.86 125.39) (end 577.87 126.4) (width 0.5) (layer F.Cu) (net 6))
 (segment (start 576.86 124.59) (end 576.86 125.39) (width 0.5) (layer F.Cu) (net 6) (status 10))
 (segment (start 577.87 126.4) (end 581.76 126.4) (width 0.5) (layer F.Cu) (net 6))
 (segment (start 581.76 102.6468) (end 589.914 94.4928) (width 0.5) (layer F.Cu) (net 6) (status 20))
 (segment (start 581.76 126.4) (end 581.76 102.6468) (width 0.5) (layer F.Cu) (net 6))
 (segment (start 589.914 90.9678) (end 589.914 91.6928) (width 1) (layer F.Cu) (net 4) (status 20))
 (segment (start 589.914 90.27248) (end 589.914 90.9678) (width 1) (layer F.Cu) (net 4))
 (segment (start 591.70149 88.48499) (end 589.914 90.27248) (width 1) (layer F.Cu) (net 4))
 (segment (start 595.51199 88.48499) (end 591.70149 88.48499) (width 1) (layer F.Cu) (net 4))
 (segment (start 596.778 89.751) (end 595.51199 88.48499) (width 1) (layer F.Cu) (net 4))
 (segment (start 600.328 89.751) (end 596.778 89.751) (width 1) (layer F.Cu) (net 4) (status 10))
 (segment (start 549.11 59.435) (end 549.11 58.87) (width 0.5) (layer F.Cu) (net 4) (status 30))
 (segment (start 549.11 58.07) (end 549.31 57.87) (width 0.5) (layer F.Cu) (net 4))
 (segment (start 549.11 58.87) (end 549.11 58.07) (width 0.5) (layer F.Cu) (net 4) (status 10))
 (segment (start 549.31 57.87) (end 556.93 57.87) (width 0.5) (layer F.Cu) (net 4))
 (segment (start 556.93 58.7088) (end 567.9 69.6788) (width 0.5) (layer F.Cu) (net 4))
 (segment (start 556.93 57.87) (end 556.93 58.7088) (width 0.5) (layer F.Cu) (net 4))
 (segment (start 567.9 69.6788) (end 567.9 78.29) (width 0.5) (layer F.Cu) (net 4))
 (segment (start 581.3028 91.6928) (end 589.914 91.6928) (width 0.5) (layer F.Cu) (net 4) (status 20))
 (segment (start 567.9 78.29) (end 581.3028 91.6928) (width 0.5) (layer F.Cu) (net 4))
 (segment (start 601.12 94.693) (end 600.328 93.901) (width 1) (layer F.Cu) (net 22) (status 30))
 (segment (start 601.12 95.86) (end 601.12 94.693) (width 1) (layer F.Cu) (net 22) (status 30))
 (segment (start 598.953 93.901) (end 600.328 93.901) (width 1) (layer F.Cu) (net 22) (status 30))
 (segment (start 596.617 91.565) (end 598.953 93.901) (width 1) (layer F.Cu) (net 22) (status 20))
 (segment (start 594.97 91.565) (end 596.617 91.565) (width 1) (layer F.Cu) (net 22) (status 10))
 (segment (start 569.4 107.58) (end 569.4 108.33) (width 0.5) (layer F.Cu) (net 1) (status 30))
 (segment (start 569.4 108.33) (end 569.4 109.13) (width 0.5) (layer F.Cu) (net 1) (status 30))
 (segment (start 569.4 113.39) (end 569.4 109.13) (width 0.5) (layer F.Cu) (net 1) (status 20))
 (segment (start 576.86 121.65) (end 576.86 120.85) (width 0.5) (layer F.Cu) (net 1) (status 10))
 (segment (start 576.86 120.85) (end 569.4 113.39) (width 0.5) (layer F.Cu) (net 1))
 (segment (start 569.4 106.755) (end 569.4 106.19) (width 0.5) (layer F.Cu) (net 2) (status 30))
 (segment (start 562.31 94.02) (end 562.31 93.5) (width 0.5) (layer F.Cu) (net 2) (status 20))
 (segment (start 562.31 98.3) (end 562.31 94.02) (width 0.5) (layer F.Cu) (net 2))
 (segment (start 569.4 106.19) (end 569.4 105.39) (width 0.5) (layer F.Cu) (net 2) (status 10))
 (segment (start 569.4 105.39) (end 562.31 98.3) (width 0.5) (layer F.Cu) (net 2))
 (segment (start 562.31 91.125) (end 562.31 90.56) (width 0.5) (layer F.Cu) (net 5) (status 30))
 (segment (start 555.55 83) (end 555.55 77.71) (width 0.5) (layer F.Cu) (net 5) (status 20))
 (segment (start 562.31 90.56) (end 562.31 89.76) (width 0.5) (layer F.Cu) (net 5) (status 10))
 (segment (start 562.31 89.76) (end 555.55 83) (width 0.5) (layer F.Cu) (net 5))
 (segment (start 549.11 67.53) (end 549.11 61.81) (width 0.5) (layer F.Cu) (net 3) (status 20))
 (segment (start 555.55 74.77) (end 555.55 73.97) (width 0.5) (layer F.Cu) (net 3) (status 10))
 (segment (start 555.55 73.97) (end 549.11 67.53) (width 0.5) (layer F.Cu) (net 3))
 (segment (start 549.11 61.81) (end 549.11 61.01) (width 0.5) (layer F.Cu) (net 3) (status 30))
 (segment (start 549.11 61.01) (end 549.11 60.26) (width 0.5) (layer F.Cu) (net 3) (status 30))
 (segment (start 591.97 90.56) (end 591.97 91.565) (width 0.5) (layer F.Cu) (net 21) (status 20))
 (segment (start 592.72 89.81) (end 591.97 90.56) (width 0.5) (layer F.Cu) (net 21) (status 10)))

